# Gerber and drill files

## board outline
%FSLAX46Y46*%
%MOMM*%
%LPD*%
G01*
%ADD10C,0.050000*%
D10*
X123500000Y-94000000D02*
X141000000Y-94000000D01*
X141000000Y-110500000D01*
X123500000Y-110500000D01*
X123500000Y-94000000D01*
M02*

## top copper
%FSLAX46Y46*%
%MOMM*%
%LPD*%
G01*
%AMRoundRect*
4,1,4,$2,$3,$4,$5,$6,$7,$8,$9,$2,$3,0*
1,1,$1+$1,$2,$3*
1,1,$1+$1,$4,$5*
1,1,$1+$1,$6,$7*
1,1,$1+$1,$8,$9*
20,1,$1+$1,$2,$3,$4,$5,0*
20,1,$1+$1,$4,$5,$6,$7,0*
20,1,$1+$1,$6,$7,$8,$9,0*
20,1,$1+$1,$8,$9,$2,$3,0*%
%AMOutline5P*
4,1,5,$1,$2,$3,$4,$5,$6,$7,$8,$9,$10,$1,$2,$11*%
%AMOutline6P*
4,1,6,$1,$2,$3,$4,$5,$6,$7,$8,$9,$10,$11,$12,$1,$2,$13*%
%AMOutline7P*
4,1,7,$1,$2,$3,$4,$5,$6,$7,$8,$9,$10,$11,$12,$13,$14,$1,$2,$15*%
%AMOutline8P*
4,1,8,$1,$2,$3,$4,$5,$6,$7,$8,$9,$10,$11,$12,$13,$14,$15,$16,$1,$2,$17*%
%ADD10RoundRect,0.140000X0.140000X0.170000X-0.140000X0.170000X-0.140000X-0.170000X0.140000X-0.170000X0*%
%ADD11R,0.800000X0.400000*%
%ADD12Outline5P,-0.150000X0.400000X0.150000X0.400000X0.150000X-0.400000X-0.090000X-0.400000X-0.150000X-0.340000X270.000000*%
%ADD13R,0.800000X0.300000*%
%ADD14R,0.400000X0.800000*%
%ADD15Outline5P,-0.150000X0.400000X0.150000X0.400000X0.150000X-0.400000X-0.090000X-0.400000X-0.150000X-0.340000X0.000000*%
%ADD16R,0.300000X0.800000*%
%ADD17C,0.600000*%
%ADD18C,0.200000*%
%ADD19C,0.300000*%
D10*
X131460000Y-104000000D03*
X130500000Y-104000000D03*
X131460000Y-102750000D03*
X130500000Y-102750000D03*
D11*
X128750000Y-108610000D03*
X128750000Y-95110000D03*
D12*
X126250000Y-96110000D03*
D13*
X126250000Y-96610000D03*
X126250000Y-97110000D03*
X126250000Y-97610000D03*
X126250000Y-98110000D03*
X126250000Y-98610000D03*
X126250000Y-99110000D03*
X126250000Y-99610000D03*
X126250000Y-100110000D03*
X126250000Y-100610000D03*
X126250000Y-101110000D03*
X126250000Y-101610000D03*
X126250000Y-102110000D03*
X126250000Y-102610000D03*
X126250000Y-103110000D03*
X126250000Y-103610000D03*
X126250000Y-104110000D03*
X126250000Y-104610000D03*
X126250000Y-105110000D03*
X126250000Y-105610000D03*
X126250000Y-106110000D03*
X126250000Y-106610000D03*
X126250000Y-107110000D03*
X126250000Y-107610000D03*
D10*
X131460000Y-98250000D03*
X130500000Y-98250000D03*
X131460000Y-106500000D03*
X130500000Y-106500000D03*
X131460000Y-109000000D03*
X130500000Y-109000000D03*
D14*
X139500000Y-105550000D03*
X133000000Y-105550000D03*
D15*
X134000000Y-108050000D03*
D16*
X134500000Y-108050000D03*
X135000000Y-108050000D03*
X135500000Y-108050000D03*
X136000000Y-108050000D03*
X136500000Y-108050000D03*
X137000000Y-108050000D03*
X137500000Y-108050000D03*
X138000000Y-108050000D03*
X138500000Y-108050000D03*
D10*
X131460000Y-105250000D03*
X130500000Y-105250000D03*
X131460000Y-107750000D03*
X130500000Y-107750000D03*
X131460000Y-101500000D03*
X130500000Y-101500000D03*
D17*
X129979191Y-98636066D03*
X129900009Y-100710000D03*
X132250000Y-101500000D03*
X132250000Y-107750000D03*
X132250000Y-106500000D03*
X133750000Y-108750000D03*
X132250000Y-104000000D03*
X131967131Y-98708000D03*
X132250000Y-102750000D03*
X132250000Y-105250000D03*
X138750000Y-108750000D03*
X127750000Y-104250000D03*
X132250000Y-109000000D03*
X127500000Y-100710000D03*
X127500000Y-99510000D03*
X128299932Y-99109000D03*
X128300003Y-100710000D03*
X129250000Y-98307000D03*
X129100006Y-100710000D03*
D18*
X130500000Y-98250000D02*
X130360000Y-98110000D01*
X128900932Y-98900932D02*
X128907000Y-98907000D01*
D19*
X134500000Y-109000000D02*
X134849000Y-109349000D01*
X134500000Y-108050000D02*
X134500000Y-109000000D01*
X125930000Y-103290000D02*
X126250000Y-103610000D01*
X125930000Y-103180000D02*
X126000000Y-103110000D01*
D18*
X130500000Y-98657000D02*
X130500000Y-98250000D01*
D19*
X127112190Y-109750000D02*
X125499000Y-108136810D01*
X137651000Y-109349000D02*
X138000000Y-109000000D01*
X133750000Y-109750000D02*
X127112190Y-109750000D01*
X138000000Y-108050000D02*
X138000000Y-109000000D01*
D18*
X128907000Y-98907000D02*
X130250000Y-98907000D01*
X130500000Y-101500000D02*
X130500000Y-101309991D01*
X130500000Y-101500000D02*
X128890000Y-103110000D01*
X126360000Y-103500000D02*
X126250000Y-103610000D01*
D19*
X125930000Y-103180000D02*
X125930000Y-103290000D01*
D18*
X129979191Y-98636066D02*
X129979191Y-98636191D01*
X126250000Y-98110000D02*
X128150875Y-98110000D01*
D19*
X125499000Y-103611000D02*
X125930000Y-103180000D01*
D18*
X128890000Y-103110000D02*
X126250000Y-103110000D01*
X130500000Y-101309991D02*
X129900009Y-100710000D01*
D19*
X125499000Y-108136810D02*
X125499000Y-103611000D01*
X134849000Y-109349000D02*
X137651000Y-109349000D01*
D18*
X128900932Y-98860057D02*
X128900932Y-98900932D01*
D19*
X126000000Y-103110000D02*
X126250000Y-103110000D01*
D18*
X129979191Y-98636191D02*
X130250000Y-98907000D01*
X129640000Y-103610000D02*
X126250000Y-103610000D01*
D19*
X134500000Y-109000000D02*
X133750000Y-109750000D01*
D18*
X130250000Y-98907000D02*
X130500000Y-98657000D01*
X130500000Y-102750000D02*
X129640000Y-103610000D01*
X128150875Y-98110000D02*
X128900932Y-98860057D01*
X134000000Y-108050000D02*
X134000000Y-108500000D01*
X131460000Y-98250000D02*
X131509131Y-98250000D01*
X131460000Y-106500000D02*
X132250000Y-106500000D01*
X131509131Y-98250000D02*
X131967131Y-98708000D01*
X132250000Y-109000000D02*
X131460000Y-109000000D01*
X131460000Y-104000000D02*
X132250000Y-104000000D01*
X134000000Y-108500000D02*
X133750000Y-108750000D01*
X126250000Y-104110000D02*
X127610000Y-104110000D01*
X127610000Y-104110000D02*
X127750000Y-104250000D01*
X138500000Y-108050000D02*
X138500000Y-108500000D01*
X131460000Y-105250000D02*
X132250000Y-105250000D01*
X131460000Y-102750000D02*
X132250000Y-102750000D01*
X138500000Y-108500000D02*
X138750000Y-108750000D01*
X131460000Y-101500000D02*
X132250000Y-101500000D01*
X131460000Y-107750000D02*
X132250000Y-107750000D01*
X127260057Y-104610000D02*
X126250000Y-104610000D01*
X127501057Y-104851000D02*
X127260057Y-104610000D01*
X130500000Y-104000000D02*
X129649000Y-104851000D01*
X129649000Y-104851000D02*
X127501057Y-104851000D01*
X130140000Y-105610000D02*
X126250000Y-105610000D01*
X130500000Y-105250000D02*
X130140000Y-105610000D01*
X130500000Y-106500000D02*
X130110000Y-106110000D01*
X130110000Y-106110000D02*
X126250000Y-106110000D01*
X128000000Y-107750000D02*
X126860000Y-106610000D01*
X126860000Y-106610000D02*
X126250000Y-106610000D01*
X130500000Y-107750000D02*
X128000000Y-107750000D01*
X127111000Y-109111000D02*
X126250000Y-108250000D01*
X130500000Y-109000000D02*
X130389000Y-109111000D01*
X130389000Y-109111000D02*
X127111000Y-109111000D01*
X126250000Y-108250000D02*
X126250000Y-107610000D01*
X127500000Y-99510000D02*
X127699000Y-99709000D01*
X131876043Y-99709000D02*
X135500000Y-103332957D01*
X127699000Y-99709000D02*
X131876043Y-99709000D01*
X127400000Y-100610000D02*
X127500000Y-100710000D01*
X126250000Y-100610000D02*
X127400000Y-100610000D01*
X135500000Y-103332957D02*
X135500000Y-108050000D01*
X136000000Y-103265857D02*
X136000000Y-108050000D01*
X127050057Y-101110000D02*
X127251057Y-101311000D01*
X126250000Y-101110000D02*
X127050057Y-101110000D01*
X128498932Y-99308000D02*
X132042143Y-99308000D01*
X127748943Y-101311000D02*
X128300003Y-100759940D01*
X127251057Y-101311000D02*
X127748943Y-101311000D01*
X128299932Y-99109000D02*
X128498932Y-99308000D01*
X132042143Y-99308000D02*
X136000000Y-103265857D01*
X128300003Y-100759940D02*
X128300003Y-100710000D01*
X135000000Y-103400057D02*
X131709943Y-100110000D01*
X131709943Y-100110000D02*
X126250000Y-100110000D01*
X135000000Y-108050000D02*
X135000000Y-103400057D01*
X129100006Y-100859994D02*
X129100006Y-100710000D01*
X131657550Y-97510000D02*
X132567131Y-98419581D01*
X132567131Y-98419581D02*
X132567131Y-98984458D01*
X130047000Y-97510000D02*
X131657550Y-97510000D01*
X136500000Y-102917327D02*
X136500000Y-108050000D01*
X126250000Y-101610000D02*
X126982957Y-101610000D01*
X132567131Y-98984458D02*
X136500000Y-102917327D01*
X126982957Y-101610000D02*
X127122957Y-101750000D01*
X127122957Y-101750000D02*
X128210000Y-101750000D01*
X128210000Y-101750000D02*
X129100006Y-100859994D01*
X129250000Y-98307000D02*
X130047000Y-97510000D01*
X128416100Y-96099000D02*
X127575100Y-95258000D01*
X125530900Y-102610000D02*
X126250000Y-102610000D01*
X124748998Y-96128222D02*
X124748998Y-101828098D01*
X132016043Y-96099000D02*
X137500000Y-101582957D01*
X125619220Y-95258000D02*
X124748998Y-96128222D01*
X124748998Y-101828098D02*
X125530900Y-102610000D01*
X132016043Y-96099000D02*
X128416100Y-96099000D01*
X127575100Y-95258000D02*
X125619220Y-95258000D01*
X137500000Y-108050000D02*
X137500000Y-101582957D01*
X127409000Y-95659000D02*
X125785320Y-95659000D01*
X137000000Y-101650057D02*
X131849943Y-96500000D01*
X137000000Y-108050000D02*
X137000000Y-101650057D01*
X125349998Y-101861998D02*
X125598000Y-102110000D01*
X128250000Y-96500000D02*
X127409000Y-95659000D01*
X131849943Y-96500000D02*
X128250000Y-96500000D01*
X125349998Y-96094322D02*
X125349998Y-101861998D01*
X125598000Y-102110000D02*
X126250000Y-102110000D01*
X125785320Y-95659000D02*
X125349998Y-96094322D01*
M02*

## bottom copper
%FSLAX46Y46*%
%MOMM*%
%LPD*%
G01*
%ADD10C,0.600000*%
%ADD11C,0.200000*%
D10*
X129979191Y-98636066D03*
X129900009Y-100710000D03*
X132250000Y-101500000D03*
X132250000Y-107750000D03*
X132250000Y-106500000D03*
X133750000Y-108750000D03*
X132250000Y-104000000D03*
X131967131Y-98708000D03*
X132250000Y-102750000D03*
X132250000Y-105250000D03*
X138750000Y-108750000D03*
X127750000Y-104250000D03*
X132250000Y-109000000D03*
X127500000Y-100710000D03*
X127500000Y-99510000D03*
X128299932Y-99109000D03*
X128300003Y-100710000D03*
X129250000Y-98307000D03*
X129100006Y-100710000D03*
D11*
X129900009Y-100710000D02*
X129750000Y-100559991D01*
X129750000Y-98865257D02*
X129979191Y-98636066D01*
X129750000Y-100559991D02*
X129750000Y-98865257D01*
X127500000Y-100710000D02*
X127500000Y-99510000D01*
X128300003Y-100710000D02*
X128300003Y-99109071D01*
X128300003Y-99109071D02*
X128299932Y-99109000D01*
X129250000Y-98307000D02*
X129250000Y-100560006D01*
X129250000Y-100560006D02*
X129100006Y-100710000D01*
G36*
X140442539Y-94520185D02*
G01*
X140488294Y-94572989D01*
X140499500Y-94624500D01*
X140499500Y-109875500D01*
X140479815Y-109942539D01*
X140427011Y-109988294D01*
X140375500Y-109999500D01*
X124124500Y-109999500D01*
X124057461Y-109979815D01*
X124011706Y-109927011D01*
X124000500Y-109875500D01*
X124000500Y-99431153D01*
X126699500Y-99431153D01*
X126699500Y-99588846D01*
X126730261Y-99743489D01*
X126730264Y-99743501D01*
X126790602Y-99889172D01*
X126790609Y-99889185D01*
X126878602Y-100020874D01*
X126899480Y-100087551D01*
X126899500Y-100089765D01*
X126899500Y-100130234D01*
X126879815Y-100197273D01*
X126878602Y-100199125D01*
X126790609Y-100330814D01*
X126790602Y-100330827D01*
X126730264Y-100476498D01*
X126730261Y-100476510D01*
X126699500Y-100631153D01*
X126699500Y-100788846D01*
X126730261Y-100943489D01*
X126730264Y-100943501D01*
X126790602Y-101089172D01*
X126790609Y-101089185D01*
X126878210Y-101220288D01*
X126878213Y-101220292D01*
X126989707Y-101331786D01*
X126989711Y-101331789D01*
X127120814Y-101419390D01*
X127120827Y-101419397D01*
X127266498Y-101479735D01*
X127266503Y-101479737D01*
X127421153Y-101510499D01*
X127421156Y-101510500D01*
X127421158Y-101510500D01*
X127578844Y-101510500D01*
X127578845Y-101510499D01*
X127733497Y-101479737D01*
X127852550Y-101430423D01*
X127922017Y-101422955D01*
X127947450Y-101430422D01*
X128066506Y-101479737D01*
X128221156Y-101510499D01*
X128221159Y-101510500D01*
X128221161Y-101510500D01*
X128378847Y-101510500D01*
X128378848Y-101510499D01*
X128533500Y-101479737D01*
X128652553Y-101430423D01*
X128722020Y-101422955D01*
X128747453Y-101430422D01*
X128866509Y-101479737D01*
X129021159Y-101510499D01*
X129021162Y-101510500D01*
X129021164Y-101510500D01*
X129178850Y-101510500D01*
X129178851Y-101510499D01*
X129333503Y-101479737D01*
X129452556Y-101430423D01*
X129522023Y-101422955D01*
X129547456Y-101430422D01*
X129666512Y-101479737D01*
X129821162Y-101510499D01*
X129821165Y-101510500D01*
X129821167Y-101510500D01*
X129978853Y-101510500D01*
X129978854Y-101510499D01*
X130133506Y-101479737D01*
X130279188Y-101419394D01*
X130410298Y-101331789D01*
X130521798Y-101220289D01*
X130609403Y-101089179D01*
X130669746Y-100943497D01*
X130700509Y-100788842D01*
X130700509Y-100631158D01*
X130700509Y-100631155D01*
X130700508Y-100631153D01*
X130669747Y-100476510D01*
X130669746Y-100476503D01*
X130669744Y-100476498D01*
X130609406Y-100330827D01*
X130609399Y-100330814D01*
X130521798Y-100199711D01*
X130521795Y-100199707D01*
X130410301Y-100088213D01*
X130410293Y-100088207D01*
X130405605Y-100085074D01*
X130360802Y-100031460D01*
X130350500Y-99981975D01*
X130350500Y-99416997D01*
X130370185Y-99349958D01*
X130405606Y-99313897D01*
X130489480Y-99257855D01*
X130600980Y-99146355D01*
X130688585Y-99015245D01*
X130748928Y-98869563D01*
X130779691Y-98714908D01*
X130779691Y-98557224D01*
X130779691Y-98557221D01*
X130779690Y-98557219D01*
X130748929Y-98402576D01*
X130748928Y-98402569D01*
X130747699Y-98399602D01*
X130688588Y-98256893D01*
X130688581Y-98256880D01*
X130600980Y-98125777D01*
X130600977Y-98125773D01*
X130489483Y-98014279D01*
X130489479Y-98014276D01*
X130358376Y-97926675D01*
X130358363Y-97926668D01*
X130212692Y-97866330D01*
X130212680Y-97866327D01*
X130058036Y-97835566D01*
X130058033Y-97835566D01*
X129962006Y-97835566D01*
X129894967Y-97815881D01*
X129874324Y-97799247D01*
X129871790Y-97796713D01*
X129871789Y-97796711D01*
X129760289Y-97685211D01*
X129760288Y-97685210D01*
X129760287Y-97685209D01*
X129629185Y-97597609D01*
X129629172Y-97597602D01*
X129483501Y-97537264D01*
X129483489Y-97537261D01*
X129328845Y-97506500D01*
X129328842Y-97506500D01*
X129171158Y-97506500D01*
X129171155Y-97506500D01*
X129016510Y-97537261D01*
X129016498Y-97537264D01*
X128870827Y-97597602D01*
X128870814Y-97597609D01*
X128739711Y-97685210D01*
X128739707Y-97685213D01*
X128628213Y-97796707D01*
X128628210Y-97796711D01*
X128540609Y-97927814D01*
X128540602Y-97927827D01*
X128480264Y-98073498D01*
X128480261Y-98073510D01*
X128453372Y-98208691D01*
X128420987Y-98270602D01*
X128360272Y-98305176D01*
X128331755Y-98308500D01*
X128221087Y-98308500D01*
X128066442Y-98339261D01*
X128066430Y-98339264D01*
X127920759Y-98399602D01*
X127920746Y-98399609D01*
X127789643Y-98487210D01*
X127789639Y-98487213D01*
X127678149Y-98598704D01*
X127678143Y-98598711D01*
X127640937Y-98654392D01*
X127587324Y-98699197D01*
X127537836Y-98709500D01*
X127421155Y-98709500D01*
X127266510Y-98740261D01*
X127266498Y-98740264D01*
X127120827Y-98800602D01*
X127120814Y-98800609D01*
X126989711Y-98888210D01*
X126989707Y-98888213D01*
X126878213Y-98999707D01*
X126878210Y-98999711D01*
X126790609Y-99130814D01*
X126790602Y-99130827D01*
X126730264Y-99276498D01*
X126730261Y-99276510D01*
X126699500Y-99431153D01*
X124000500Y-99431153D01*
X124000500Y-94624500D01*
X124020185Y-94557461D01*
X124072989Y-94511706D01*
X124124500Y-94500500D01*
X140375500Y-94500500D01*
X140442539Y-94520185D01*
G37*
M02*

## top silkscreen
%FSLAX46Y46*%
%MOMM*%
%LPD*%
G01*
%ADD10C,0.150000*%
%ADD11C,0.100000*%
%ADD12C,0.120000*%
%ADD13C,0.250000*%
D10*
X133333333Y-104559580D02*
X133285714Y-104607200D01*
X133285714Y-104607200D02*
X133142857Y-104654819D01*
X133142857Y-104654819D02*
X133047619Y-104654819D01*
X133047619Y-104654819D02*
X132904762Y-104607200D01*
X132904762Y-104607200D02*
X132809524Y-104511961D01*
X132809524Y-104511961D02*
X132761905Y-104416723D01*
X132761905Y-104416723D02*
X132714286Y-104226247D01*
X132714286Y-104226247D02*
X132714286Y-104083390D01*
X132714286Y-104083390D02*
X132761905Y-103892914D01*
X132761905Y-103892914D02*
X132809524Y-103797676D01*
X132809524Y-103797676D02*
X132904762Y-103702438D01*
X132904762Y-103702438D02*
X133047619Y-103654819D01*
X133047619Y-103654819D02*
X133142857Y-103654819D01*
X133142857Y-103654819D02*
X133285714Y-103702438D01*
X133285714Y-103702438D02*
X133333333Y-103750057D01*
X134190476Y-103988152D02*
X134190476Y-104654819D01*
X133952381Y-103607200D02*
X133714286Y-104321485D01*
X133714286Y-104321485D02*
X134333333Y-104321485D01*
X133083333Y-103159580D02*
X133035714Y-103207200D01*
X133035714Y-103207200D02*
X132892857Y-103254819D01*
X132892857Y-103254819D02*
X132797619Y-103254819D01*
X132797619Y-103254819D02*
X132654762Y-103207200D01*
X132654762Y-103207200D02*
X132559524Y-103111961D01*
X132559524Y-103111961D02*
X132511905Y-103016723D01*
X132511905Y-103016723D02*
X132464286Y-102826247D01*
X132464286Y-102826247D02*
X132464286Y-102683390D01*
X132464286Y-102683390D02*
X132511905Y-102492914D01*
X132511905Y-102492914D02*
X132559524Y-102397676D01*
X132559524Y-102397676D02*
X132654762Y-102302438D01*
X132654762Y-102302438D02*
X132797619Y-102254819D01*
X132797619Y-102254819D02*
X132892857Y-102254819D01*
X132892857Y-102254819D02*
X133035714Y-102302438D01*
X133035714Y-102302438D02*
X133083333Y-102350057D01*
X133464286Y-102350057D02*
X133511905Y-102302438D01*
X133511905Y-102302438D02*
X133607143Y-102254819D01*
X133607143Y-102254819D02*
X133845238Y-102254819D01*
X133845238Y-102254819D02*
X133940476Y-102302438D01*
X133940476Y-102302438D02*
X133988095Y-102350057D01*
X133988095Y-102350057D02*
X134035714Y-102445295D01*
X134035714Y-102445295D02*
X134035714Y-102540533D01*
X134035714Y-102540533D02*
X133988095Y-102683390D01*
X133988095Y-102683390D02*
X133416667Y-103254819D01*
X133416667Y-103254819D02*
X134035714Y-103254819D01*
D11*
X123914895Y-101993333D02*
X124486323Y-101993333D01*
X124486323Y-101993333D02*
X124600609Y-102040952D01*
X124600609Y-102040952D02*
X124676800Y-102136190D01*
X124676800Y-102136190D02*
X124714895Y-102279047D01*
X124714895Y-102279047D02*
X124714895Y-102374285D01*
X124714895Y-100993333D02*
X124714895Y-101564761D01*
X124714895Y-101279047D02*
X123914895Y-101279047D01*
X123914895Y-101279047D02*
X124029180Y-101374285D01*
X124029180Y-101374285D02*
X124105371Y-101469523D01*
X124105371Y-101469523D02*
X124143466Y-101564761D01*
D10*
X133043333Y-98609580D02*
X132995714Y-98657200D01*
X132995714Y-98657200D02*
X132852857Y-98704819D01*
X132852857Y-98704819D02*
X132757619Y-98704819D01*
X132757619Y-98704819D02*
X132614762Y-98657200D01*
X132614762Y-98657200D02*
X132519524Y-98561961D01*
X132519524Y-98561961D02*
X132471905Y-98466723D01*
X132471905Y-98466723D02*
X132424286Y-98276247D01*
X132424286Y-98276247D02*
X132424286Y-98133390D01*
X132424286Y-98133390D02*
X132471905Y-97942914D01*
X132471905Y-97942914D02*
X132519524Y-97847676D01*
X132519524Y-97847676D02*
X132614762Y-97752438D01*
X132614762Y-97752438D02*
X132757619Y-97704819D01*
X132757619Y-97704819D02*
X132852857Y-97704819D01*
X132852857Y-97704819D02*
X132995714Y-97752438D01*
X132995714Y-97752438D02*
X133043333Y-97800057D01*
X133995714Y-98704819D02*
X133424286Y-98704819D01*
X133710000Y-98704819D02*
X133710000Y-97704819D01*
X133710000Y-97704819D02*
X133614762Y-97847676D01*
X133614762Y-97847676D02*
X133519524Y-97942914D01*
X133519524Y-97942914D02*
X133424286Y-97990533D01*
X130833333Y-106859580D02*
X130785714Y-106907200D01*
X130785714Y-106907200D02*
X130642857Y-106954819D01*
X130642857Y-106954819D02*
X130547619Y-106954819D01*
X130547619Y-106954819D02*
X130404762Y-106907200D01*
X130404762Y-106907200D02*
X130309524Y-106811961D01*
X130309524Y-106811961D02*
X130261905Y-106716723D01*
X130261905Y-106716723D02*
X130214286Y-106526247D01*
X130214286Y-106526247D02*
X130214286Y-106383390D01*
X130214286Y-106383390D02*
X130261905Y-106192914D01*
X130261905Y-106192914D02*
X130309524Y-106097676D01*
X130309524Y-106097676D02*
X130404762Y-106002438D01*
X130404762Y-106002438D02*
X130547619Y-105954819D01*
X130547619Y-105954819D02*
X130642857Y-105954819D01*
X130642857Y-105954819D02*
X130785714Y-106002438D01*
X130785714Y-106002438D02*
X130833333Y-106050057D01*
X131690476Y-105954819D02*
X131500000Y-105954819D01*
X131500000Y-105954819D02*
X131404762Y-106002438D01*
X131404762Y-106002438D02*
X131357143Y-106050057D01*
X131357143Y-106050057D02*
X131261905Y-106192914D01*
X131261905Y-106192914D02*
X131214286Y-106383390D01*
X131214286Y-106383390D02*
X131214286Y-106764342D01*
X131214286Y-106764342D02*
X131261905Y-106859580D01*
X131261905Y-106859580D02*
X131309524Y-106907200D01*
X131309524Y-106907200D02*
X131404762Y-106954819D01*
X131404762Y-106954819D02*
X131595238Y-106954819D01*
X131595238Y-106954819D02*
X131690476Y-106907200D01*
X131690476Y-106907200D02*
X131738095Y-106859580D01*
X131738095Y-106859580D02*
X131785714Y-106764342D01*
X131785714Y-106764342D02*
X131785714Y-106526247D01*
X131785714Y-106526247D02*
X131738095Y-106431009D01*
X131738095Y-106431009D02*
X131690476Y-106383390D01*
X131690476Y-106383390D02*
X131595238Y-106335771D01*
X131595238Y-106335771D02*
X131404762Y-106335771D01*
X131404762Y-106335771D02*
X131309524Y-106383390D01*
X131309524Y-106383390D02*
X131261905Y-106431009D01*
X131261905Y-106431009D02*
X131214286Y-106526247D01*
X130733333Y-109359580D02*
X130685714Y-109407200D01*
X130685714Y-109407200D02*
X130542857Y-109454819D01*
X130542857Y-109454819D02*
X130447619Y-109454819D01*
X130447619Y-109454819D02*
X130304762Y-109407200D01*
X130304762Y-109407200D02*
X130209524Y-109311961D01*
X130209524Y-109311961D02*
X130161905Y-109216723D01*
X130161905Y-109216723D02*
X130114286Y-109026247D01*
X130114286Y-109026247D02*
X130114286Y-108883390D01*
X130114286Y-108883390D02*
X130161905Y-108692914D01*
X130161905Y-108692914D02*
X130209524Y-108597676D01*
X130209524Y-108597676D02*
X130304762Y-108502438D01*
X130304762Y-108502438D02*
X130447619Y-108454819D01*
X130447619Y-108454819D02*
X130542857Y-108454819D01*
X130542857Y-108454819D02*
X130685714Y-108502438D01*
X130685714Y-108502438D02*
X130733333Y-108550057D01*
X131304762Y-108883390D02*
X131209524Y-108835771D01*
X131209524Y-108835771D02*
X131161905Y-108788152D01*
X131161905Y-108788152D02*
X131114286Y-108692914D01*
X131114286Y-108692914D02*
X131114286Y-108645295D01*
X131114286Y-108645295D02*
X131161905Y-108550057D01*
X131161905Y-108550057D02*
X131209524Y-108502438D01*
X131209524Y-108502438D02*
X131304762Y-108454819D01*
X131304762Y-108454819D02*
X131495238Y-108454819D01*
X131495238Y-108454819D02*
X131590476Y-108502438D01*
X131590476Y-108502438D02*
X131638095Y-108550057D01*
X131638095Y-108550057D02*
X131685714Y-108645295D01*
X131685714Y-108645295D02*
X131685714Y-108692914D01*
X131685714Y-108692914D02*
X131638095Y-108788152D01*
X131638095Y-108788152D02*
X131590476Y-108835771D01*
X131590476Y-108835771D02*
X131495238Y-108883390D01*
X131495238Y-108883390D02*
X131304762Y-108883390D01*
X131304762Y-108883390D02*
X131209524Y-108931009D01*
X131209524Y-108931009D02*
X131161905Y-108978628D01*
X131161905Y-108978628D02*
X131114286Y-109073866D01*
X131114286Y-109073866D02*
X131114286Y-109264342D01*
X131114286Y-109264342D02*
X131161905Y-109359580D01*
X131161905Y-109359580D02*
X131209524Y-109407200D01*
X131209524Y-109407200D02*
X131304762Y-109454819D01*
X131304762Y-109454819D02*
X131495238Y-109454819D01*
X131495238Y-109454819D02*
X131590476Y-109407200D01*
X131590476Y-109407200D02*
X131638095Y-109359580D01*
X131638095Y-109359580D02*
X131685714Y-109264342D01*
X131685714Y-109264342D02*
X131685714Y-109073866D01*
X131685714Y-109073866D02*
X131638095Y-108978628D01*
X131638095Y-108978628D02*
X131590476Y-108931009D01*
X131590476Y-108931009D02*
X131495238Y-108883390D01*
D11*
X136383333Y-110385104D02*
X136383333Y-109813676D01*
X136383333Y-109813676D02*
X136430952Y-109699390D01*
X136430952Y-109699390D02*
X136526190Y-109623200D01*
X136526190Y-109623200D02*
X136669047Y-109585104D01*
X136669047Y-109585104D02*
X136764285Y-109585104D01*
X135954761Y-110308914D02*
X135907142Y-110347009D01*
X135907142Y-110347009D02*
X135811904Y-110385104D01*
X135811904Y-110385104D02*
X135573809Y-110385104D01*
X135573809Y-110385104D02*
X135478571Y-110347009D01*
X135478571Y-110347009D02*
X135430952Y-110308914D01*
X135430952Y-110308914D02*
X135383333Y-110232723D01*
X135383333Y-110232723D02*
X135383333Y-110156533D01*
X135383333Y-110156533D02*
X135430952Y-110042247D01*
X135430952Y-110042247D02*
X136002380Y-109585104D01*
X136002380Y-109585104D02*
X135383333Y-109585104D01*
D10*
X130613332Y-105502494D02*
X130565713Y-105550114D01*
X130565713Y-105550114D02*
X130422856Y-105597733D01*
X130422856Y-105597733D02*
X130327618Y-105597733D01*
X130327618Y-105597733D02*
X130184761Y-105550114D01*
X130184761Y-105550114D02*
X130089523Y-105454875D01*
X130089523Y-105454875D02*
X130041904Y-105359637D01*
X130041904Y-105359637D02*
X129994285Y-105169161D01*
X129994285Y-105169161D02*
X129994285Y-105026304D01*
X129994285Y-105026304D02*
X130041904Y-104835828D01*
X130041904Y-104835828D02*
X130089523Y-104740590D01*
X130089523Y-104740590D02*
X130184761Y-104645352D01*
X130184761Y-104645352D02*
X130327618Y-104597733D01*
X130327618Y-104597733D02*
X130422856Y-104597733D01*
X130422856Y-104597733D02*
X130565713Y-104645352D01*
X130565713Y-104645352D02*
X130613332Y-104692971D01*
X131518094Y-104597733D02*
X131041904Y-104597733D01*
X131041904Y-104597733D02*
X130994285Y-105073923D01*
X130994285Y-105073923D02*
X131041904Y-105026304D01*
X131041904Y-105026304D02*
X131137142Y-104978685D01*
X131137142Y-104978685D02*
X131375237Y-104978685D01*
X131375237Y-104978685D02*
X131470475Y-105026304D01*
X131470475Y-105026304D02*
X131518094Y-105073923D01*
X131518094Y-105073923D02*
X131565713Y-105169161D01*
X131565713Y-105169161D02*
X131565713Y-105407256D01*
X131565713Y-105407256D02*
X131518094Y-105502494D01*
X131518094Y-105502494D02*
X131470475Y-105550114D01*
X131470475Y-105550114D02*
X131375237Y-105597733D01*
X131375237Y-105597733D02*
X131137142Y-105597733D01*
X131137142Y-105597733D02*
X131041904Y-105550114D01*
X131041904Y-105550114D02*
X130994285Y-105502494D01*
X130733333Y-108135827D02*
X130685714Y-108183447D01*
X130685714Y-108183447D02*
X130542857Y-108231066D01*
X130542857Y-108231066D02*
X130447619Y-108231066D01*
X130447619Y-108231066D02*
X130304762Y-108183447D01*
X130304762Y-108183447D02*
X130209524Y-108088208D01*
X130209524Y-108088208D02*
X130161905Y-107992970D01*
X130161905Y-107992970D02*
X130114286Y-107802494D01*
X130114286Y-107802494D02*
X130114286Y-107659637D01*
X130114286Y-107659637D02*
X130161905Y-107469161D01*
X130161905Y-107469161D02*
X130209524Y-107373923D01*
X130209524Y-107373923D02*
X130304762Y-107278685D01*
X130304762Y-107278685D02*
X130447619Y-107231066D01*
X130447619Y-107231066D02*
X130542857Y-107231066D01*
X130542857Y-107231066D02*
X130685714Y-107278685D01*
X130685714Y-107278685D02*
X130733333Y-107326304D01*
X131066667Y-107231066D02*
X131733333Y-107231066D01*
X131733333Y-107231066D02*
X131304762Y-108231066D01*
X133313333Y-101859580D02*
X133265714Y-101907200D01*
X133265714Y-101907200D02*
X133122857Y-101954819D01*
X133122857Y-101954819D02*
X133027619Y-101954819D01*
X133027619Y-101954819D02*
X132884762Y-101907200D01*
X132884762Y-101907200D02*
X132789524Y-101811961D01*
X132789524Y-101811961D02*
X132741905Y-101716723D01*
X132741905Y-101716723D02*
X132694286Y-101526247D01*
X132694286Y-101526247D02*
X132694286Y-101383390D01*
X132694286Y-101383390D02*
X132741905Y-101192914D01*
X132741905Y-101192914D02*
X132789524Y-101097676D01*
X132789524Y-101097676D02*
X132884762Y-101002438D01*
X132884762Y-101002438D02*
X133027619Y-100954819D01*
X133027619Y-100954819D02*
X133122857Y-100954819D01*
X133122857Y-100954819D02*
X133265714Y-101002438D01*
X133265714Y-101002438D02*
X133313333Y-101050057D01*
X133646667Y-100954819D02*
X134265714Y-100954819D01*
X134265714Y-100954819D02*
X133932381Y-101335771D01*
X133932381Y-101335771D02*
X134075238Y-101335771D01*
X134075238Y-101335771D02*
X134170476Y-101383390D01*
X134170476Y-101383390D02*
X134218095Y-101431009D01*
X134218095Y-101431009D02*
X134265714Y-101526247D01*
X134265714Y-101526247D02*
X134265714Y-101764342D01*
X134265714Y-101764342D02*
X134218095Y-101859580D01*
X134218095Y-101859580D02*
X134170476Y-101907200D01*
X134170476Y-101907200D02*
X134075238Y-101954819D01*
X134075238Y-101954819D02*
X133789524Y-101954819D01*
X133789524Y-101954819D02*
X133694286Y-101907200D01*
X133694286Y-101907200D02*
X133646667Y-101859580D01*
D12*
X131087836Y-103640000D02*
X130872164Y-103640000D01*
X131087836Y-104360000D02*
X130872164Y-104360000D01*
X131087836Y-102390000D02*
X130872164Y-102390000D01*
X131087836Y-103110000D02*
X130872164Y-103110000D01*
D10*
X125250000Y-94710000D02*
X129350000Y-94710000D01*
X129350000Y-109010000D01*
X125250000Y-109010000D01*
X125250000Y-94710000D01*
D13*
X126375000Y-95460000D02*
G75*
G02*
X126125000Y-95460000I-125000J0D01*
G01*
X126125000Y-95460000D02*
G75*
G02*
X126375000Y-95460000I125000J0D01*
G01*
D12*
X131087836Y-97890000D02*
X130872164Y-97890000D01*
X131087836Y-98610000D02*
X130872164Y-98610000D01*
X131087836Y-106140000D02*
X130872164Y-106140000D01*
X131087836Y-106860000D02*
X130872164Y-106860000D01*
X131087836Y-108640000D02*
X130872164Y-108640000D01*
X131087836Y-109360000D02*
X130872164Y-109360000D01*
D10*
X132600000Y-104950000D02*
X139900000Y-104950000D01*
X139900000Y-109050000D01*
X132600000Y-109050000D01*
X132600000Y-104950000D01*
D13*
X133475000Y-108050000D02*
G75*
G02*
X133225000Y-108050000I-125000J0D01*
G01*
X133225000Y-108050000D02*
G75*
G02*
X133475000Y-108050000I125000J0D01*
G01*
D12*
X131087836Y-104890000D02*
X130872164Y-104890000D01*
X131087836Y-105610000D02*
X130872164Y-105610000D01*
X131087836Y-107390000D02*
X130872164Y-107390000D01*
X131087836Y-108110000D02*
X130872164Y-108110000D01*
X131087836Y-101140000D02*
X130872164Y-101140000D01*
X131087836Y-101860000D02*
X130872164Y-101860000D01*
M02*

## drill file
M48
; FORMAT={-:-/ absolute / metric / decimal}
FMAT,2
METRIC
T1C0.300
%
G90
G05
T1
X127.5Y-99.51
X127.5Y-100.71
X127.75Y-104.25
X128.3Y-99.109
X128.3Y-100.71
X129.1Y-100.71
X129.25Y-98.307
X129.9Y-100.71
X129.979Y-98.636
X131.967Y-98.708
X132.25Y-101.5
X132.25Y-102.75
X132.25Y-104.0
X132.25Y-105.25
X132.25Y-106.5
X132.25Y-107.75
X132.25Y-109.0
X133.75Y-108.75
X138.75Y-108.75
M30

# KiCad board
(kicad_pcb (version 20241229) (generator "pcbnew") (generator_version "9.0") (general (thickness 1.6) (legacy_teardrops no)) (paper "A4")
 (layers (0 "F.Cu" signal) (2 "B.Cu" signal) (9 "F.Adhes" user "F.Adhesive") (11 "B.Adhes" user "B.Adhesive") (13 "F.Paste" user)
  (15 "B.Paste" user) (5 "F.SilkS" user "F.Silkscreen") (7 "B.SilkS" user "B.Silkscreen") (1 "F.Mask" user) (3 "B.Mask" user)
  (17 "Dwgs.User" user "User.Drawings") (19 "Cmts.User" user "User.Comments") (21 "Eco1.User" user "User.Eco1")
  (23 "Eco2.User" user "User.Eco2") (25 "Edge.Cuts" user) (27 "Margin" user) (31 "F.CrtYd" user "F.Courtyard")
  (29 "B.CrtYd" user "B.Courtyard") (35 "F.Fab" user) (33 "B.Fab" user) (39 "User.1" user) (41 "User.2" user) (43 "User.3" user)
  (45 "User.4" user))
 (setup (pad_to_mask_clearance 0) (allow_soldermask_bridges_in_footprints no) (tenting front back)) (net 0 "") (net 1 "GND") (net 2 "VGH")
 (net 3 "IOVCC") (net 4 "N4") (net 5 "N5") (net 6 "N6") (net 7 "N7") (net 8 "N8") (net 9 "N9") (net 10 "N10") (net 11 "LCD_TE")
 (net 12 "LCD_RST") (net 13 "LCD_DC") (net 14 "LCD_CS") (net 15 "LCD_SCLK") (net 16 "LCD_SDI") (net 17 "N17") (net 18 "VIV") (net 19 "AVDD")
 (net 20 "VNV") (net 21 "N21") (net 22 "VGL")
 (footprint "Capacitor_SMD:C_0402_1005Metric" (layer "F.Cu") (at 130.98 104 180)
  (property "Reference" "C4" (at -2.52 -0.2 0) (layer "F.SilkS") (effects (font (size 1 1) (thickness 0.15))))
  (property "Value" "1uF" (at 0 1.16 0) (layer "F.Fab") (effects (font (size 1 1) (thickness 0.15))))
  (fp_line (start -0.107836 0.36) (end 0.107836 0.36) (stroke (width 0.12) (type solid)) (layer "F.SilkS"))
  (fp_line (start -0.107836 -0.36) (end 0.107836 -0.36) (stroke (width 0.12) (type solid)) (layer "F.SilkS"))
  (pad "1" smd roundrect (at -0.48 0 180) (size 0.56 0.62) (layers "F.Cu" "F.Mask" "F.Paste") (roundrect_rratio 0.25) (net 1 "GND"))
  (pad "2" smd roundrect (at 0.48 0 180) (size 0.56 0.62) (layers "F.Cu" "F.Mask" "F.Paste") (roundrect_rratio 0.25) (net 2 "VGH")))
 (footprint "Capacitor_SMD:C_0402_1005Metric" (layer "F.Cu") (at 130.98 102.75 180)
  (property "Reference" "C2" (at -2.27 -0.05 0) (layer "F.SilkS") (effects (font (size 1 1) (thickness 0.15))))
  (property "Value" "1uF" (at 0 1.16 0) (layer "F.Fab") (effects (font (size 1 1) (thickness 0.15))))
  (fp_line (start -0.107836 0.36) (end 0.107836 0.36) (stroke (width 0.12) (type solid)) (layer "F.SilkS"))
  (fp_line (start -0.107836 -0.36) (end 0.107836 -0.36) (stroke (width 0.12) (type solid)) (layer "F.SilkS"))
  (pad "1" smd roundrect (at -0.48 0 180) (size 0.56 0.62) (layers "F.Cu" "F.Mask" "F.Paste") (roundrect_rratio 0.25) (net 1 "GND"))
  (pad "2" smd roundrect (at 0.48 0 180) (size 0.56 0.62) (layers "F.Cu" "F.Mask" "F.Paste") (roundrect_rratio 0.25) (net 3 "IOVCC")))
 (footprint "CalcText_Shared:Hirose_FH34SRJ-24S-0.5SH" (layer "F.Cu") (at 126.25 101.86 90)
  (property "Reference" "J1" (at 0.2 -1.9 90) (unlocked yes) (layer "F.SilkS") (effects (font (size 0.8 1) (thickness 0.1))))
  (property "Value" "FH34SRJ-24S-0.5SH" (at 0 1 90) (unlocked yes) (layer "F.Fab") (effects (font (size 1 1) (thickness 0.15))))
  (fp_rect (start -7.15 -1) (end 7.15 3.1) (stroke (width 0.15) (type solid)) (fill no) (layer "F.SilkS"))
  (fp_circle (center 6.4 0) (end 6.6 0) (stroke (width 0.1) (type default)) (fill yes) (layer "F.SilkS"))
  (pad "" smd rect (at -6.75 2.5 90) (size 0.4 0.8) (layers "F.Cu" "F.Mask" "F.Paste") (thermal_bridge_angle 45))
  (pad "" smd rect (at 6.75 2.5 90) (size 0.4 0.8) (layers "F.Cu" "F.Mask" "F.Paste") (thermal_bridge_angle 45))
  (pad "1" smd roundrect (at 5.75 0 270) (size 0.3 0.8) (layers "F.Cu" "F.Mask" "F.Paste") (roundrect_rratio 0) (chamfer_ratio 0.2)
   (chamfer bottom_left) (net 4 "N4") (thermal_bridge_angle 45))
  (pad "2" smd rect (at 5.25 0 270) (size 0.3 0.8) (layers "F.Cu" "F.Mask" "F.Paste") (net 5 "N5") (thermal_bridge_angle 45))
  (pad "3" smd rect (at 4.75 0 270) (size 0.3 0.8) (layers "F.Cu" "F.Mask" "F.Paste") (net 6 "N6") (thermal_bridge_angle 45))
  (pad "4" smd rect (at 4.25 0 270) (size 0.3 0.8) (layers "F.Cu" "F.Mask" "F.Paste") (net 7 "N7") (thermal_bridge_angle 45))
  (pad "5" smd rect (at 3.75 0 270) (size 0.3 0.8) (layers "F.Cu" "F.Mask" "F.Paste") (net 3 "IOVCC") (thermal_bridge_angle 45))
  (pad "6" smd rect (at 3.25 0 270) (size 0.3 0.8) (layers "F.Cu" "F.Mask" "F.Paste") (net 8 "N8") (thermal_bridge_angle 45))
  (pad "7" smd rect (at 2.75 0 270) (size 0.3 0.8) (layers "F.Cu" "F.Mask" "F.Paste") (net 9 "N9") (thermal_bridge_angle 45))
  (pad "8" smd rect (at 2.25 0 270) (size 0.3 0.8) (layers "F.Cu" "F.Mask" "F.Paste") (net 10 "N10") (thermal_bridge_angle 45))
  (pad "9" smd rect (at 1.75 0 270) (size 0.3 0.8) (layers "F.Cu" "F.Mask" "F.Paste") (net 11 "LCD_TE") (thermal_bridge_angle 45))
  (pad "10" smd rect (at 1.25 0 270) (size 0.3 0.8) (layers "F.Cu" "F.Mask" "F.Paste") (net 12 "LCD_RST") (thermal_bridge_angle 45))
  (pad "11" smd rect (at 0.75 0 270) (size 0.3 0.8) (layers "F.Cu" "F.Mask" "F.Paste") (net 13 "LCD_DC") (thermal_bridge_angle 45))
  (pad "12" smd rect (at 0.25 0 270) (size 0.3 0.8) (layers "F.Cu" "F.Mask" "F.Paste") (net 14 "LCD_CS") (thermal_bridge_angle 45))
  (pad "13" smd rect (at -0.25 0 270) (size 0.3 0.8) (layers "F.Cu" "F.Mask" "F.Paste") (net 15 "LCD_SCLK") (thermal_bridge_angle 45))
  (pad "14" smd rect (at -0.75 0 270) (size 0.3 0.8) (layers "F.Cu" "F.Mask" "F.Paste") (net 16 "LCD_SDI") (thermal_bridge_angle 45))
  (pad "15" smd rect (at -1.25 0 270) (size 0.3 0.8) (layers "F.Cu" "F.Mask" "F.Paste") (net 3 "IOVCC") (thermal_bridge_angle 45))
  (pad "16" smd rect (at -1.75 0 270) (size 0.3 0.8) (layers "F.Cu" "F.Mask" "F.Paste") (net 3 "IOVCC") (thermal_bridge_angle 45))
  (pad "17" smd rect (at -2.25 0 270) (size 0.3 0.8) (layers "F.Cu" "F.Mask" "F.Paste") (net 1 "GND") (thermal_bridge_angle 45))
  (pad "18" smd rect (at -2.75 0 270) (size 0.3 0.8) (layers "F.Cu" "F.Mask" "F.Paste") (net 2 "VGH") (thermal_bridge_angle 45))
  (pad "19" smd rect (at -3.25 0 270) (size 0.3 0.8) (layers "F.Cu" "F.Mask" "F.Paste") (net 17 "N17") (thermal_bridge_angle 45))
  (pad "20" smd rect (at -3.75 0 270) (size 0.3 0.8) (layers "F.Cu" "F.Mask" "F.Paste") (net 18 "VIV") (thermal_bridge_angle 45))
  (pad "21" smd rect (at -4.25 0 270) (size 0.3 0.8) (layers "F.Cu" "F.Mask" "F.Paste") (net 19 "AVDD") (thermal_bridge_angle 45))
  (pad "22" smd rect (at -4.75 0 270) (size 0.3 0.8) (layers "F.Cu" "F.Mask" "F.Paste") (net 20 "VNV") (thermal_bridge_angle 45))
  (pad "23" smd rect (at -5.25 0 270) (size 0.3 0.8) (layers "F.Cu" "F.Mask" "F.Paste") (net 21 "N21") (thermal_bridge_angle 45))
  (pad "24" smd rect (at -5.75 0 270) (size 0.3 0.8) (layers "F.Cu" "F.Mask" "F.Paste") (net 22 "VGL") (thermal_bridge_angle 45)))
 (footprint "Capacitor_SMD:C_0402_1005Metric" (layer "F.Cu") (at 130.98 98.25 180)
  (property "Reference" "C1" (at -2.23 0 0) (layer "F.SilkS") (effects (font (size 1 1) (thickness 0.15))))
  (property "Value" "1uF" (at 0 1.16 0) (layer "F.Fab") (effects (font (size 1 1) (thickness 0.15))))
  (fp_line (start -0.107836 0.36) (end 0.107836 0.36) (stroke (width 0.12) (type solid)) (layer "F.SilkS"))
  (fp_line (start -0.107836 -0.36) (end 0.107836 -0.36) (stroke (width 0.12) (type solid)) (layer "F.SilkS"))
  (pad "1" smd roundrect (at -0.48 0 180) (size 0.56 0.62) (layers "F.Cu" "F.Mask" "F.Paste") (roundrect_rratio 0.25) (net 1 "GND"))
  (pad "2" smd roundrect (at 0.48 0 180) (size 0.56 0.62) (layers "F.Cu" "F.Mask" "F.Paste") (roundrect_rratio 0.25) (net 3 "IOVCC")))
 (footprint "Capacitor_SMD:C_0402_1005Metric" (layer "F.Cu") (at 130.98 106.5 180)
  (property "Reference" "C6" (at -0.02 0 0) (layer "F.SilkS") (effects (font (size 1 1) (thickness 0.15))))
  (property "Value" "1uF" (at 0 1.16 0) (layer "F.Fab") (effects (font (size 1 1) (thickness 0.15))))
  (fp_line (start -0.107836 0.36) (end 0.107836 0.36) (stroke (width 0.12) (type solid)) (layer "F.SilkS"))
  (fp_line (start -0.107836 -0.36) (end 0.107836 -0.36) (stroke (width 0.12) (type solid)) (layer "F.SilkS"))
  (pad "1" smd roundrect (at -0.48 0 180) (size 0.56 0.62) (layers "F.Cu" "F.Mask" "F.Paste") (roundrect_rratio 0.25) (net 1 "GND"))
  (pad "2" smd roundrect (at 0.48 0 180) (size 0.56 0.62) (layers "F.Cu" "F.Mask" "F.Paste") (roundrect_rratio 0.25) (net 19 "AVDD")))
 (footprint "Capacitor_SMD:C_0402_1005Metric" (layer "F.Cu") (at 130.98 109 180)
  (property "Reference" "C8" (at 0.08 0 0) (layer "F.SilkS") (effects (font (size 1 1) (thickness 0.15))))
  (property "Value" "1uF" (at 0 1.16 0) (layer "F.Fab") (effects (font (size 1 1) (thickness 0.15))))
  (fp_line (start -0.107836 0.36) (end 0.107836 0.36) (stroke (width 0.12) (type solid)) (layer "F.SilkS"))
  (fp_line (start -0.107836 -0.36) (end 0.107836 -0.36) (stroke (width 0.12) (type solid)) (layer "F.SilkS"))
  (pad "1" smd roundrect (at -0.48 0 180) (size 0.56 0.62) (layers "F.Cu" "F.Mask" "F.Paste") (roundrect_rratio 0.25) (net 1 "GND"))
  (pad "2" smd roundrect (at 0.48 0 180) (size 0.56 0.62) (layers "F.Cu" "F.Mask" "F.Paste") (roundrect_rratio 0.25) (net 22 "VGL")))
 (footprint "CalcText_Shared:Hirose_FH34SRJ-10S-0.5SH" (layer "F.Cu") (at 136.25 108.05 180)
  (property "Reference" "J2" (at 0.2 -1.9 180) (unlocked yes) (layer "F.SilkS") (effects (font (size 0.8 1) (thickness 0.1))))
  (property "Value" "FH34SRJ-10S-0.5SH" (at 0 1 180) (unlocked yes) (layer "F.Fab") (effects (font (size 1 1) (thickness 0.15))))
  (fp_rect (start -3.65 -1) (end 3.65 3.1) (stroke (width 0.15) (type solid)) (fill no) (layer "F.SilkS"))
  (fp_circle (center 2.9 0) (end 3.1 0) (stroke (width 0.1) (type default)) (fill yes) (layer "F.SilkS"))
  (pad "" smd rect (at -3.25 2.5 180) (size 0.4 0.8) (layers "F.Cu" "F.Mask" "F.Paste") (thermal_bridge_angle 45))
  (pad "" smd rect (at 3.25 2.5 180) (size 0.4 0.8) (layers "F.Cu" "F.Mask" "F.Paste") (thermal_bridge_angle 45))
  (pad "1" smd roundrect (at 2.25 0) (size 0.3 0.8) (layers "F.Cu" "F.Mask" "F.Paste") (roundrect_rratio 0) (chamfer_ratio 0.2)
   (chamfer bottom_left) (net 1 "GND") (thermal_bridge_angle 45))
  (pad "2" smd rect (at 1.75 0) (size 0.3 0.8) (layers "F.Cu" "F.Mask" "F.Paste") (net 3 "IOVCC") (thermal_bridge_angle 45))
  (pad "3" smd rect (at 1.25 0) (size 0.3 0.8) (layers "F.Cu" "F.Mask" "F.Paste") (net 11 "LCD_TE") (thermal_bridge_angle 45))
  (pad "4" smd rect (at 0.75 0) (size 0.3 0.8) (layers "F.Cu" "F.Mask" "F.Paste") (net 12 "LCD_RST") (thermal_bridge_angle 45))
  (pad "5" smd rect (at 0.25 0) (size 0.3 0.8) (layers "F.Cu" "F.Mask" "F.Paste") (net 13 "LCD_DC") (thermal_bridge_angle 45))
  (pad "6" smd rect (at -0.25 0) (size 0.3 0.8) (layers "F.Cu" "F.Mask" "F.Paste") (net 14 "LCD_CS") (thermal_bridge_angle 45))
  (pad "7" smd rect (at -0.75 0) (size 0.3 0.8) (layers "F.Cu" "F.Mask" "F.Paste") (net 15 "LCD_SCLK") (thermal_bridge_angle 45))
  (pad "8" smd rect (at -1.25 0) (size 0.3 0.8) (layers "F.Cu" "F.Mask" "F.Paste") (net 16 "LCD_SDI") (thermal_bridge_angle 45))
  (pad "9" smd rect (at -1.75 0) (size 0.3 0.8) (layers "F.Cu" "F.Mask" "F.Paste") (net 3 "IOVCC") (thermal_bridge_angle 45))
  (pad "10" smd rect (at -2.25 0) (size 0.3 0.8) (layers "F.Cu" "F.Mask" "F.Paste") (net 1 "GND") (thermal_bridge_angle 45)))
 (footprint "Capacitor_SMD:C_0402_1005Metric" (layer "F.Cu") (at 130.98 105.25 180)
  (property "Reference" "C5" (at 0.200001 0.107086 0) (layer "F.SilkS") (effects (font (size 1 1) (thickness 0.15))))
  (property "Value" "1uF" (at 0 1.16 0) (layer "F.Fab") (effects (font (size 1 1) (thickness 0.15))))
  (fp_line (start -0.107836 0.36) (end 0.107836 0.36) (stroke (width 0.12) (type solid)) (layer "F.SilkS"))
  (fp_line (start -0.107836 -0.36) (end 0.107836 -0.36) (stroke (width 0.12) (type solid)) (layer "F.SilkS"))
  (pad "1" smd roundrect (at -0.48 0 180) (size 0.56 0.62) (layers "F.Cu" "F.Mask" "F.Paste") (roundrect_rratio 0.25) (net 1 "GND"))
  (pad "2" smd roundrect (at 0.48 0 180) (size 0.56 0.62) (layers "F.Cu" "F.Mask" "F.Paste") (roundrect_rratio 0.25) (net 18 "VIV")))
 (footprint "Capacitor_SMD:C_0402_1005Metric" (layer "F.Cu") (at 130.98 107.75 180)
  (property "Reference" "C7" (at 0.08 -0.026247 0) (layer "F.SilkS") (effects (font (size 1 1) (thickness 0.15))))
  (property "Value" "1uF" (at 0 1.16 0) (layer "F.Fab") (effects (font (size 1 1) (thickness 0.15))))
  (fp_line (start -0.107836 0.36) (end 0.107836 0.36) (stroke (width 0.12) (type solid)) (layer "F.SilkS"))
  (fp_line (start -0.107836 -0.36) (end 0.107836 -0.36) (stroke (width 0.12) (type solid)) (layer "F.SilkS"))
  (pad "1" smd roundrect (at -0.48 0 180) (size 0.56 0.62) (layers "F.Cu" "F.Mask" "F.Paste") (roundrect_rratio 0.25) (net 1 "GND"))
  (pad "2" smd roundrect (at 0.48 0 180) (size 0.56 0.62) (layers "F.Cu" "F.Mask" "F.Paste") (roundrect_rratio 0.25) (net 20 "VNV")))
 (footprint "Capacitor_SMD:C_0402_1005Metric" (layer "F.Cu") (at 130.98 101.5 180)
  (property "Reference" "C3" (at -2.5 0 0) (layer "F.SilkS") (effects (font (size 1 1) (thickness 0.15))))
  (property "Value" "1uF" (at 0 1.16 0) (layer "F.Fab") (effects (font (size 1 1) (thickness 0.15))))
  (fp_line (start -0.107836 0.36) (end 0.107836 0.36) (stroke (width 0.12) (type solid)) (layer "F.SilkS"))
  (fp_line (start -0.107836 -0.36) (end 0.107836 -0.36) (stroke (width 0.12) (type solid)) (layer "F.SilkS"))
  (pad "1" smd roundrect (at -0.48 0 180) (size 0.56 0.62) (layers "F.Cu" "F.Mask" "F.Paste") (roundrect_rratio 0.25) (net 1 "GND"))
  (pad "2" smd roundrect (at 0.48 0 180) (size 0.56 0.62) (layers "F.Cu" "F.Mask" "F.Paste") (roundrect_rratio 0.25) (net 3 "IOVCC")))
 (gr_rect (start 123.5 94) (end 141 110.5) (stroke (width 0.05) (type default)) (fill no) (layer "Edge.Cuts"))
 (segment (start 130.5 98.25) (end 130.36 98.11) (width 0.2) (layer "F.Cu") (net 3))
 (segment (start 128.900932 98.900932) (end 128.907 98.907) (width 0.2) (layer "F.Cu") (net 3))
 (segment (start 134.5 109) (end 134.849 109.349) (width 0.3) (layer "F.Cu") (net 3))
 (segment (start 134.5 108.05) (end 134.5 109) (width 0.3) (layer "F.Cu") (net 3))
 (segment (start 125.93 103.29) (end 126.25 103.61) (width 0.3) (layer "F.Cu") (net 3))
 (segment (start 125.93 103.18) (end 126 103.11) (width 0.3) (layer "F.Cu") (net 3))
 (segment (start 130.5 98.657) (end 130.5 98.25) (width 0.2) (layer "F.Cu") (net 3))
 (segment (start 127.11219 109.75) (end 125.499 108.13681) (width 0.3) (layer "F.Cu") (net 3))
 (segment (start 137.651 109.349) (end 138 109) (width 0.3) (layer "F.Cu") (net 3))
 (segment (start 133.75 109.75) (end 127.11219 109.75) (width 0.3) (layer "F.Cu") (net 3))
 (segment (start 138 108.05) (end 138 109) (width 0.3) (layer "F.Cu") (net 3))
 (segment (start 128.907 98.907) (end 130.25 98.907) (width 0.2) (layer "F.Cu") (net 3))
 (segment (start 130.5 101.5) (end 130.5 101.309991) (width 0.2) (layer "F.Cu") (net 3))
 (segment (start 130.5 101.5) (end 128.89 103.11) (width 0.2) (layer "F.Cu") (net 3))
 (segment (start 126.36 103.5) (end 126.25 103.61) (width 0.2) (layer "F.Cu") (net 3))
 (segment (start 125.93 103.18) (end 125.93 103.29) (width 0.3) (layer "F.Cu") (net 3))
 (segment (start 129.979191 98.636066) (end 129.979191 98.636191) (width 0.2) (layer "F.Cu") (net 3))
 (segment (start 126.25 98.11) (end 128.150875 98.11) (width 0.2) (layer "F.Cu") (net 3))
 (segment (start 125.499 103.611) (end 125.93 103.18) (width 0.3) (layer "F.Cu") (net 3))
 (segment (start 128.89 103.11) (end 126.25 103.11) (width 0.2) (layer "F.Cu") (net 3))
 (segment (start 130.5 101.309991) (end 129.900009 100.71) (width 0.2) (layer "F.Cu") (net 3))
 (segment (start 125.499 108.13681) (end 125.499 103.611) (width 0.3) (layer "F.Cu") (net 3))
 (segment (start 134.849 109.349) (end 137.651 109.349) (width 0.3) (layer "F.Cu") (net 3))
 (segment (start 128.900932 98.860057) (end 128.900932 98.900932) (width 0.2) (layer "F.Cu") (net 3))
 (segment (start 126 103.11) (end 126.25 103.11) (width 0.3) (layer "F.Cu") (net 3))
 (segment (start 129.979191 98.636191) (end 130.25 98.907) (width 0.2) (layer "F.Cu") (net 3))
 (segment (start 129.64 103.61) (end 126.25 103.61) (width 0.2) (layer "F.Cu") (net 3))
 (segment (start 134.5 109) (end 133.75 109.75) (width 0.3) (layer "F.Cu") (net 3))
 (segment (start 130.25 98.907) (end 130.5 98.657) (width 0.2) (layer "F.Cu") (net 3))
 (segment (start 130.5 102.75) (end 129.64 103.61) (width 0.2) (layer "F.Cu") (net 3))
 (segment (start 128.150875 98.11) (end 128.900932 98.860057) (width 0.2) (layer "F.Cu") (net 3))
 (via (at 129.979191 98.636066) (size 0.6) (drill 0.3) (layers "F.Cu" "B.Cu") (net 3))
 (via (at 129.900009 100.71) (size 0.6) (drill 0.3) (layers "F.Cu" "B.Cu") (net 3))
 (segment (start 129.900009 100.71) (end 129.75 100.559991) (width 0.2) (layer "B.Cu") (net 3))
 (segment (start 129.75 98.865257) (end 129.979191 98.636066) (width 0.2) (layer "B.Cu") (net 3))
 (segment (start 129.75 100.559991) (end 129.75 98.865257) (width 0.2) (layer "B.Cu") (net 3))
 (segment (start 134 108.05) (end 134 108.5) (width 0.2) (layer "F.Cu") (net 1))
 (segment (start 131.46 98.25) (end 131.509131 98.25) (width 0.2) (layer "F.Cu") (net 1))
 (segment (start 131.46 106.5) (end 132.25 106.5) (width 0.2) (layer "F.Cu") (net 1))
 (segment (start 131.509131 98.25) (end 131.967131 98.708) (width 0.2) (layer "F.Cu") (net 1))
 (segment (start 132.25 109) (end 131.46 109) (width 0.2) (layer "F.Cu") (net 1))
 (segment (start 131.46 104) (end 132.25 104) (width 0.2) (layer "F.Cu") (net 1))
 (segment (start 134 108.5) (end 133.75 108.75) (width 0.2) (layer "F.Cu") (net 1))
 (segment (start 126.25 104.11) (end 127.61 104.11) (width 0.2) (layer "F.Cu") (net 1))
 (segment (start 127.61 104.11) (end 127.75 104.25) (width 0.2) (layer "F.Cu") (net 1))
 (segment (start 138.5 108.05) (end 138.5 108.5) (width 0.2) (layer "F.Cu") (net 1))
 (segment (start 131.46 105.25) (end 132.25 105.25) (width 0.2) (layer "F.Cu") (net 1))
 (segment (start 131.46 102.75) (end 132.25 102.75) (width 0.2) (layer "F.Cu") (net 1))
 (segment (start 138.5 108.5) (end 138.75 108.75) (width 0.2) (layer "F.Cu") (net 1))
 (segment (start 131.46 101.5) (end 132.25 101.5) (width 0.2) (layer "F.Cu") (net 1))
 (segment (start 131.46 107.75) (end 132.25 107.75) (width 0.2) (layer "F.Cu") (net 1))
 (via (at 132.25 101.5) (size 0.6) (drill 0.3) (layers "F.Cu" "B.Cu") (free yes) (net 1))
 (via (at 132.25 107.75) (size 0.6) (drill 0.3) (layers "F.Cu" "B.Cu") (free yes) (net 1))
 (via (at 132.25 106.5) (size 0.6) (drill 0.3) (layers "F.Cu" "B.Cu") (free yes) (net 1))
 (via (at 133.75 108.75) (size 0.6) (drill 0.3) (layers "F.Cu" "B.Cu") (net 1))
 (via (at 132.25 104) (size 0.6) (drill 0.3) (layers "F.Cu" "B.Cu") (free yes) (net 1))
 (via (at 131.967131 98.708) (size 0.6) (drill 0.3) (layers "F.Cu" "B.Cu") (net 1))
 (via (at 132.25 102.75) (size 0.6) (drill 0.3) (layers "F.Cu" "B.Cu") (free yes) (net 1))
 (via (at 132.25 105.25) (size 0.6) (drill 0.3) (layers "F.Cu" "B.Cu") (free yes) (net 1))
 (via (at 138.75 108.75) (size 0.6) (drill 0.3) (layers "F.Cu" "B.Cu") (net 1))
 (via (at 127.75 104.25) (size 0.6) (drill 0.3) (layers "F.Cu" "B.Cu") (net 1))
 (via (at 132.25 109) (size 0.6) (drill 0.3) (layers "F.Cu" "B.Cu") (free yes) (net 1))
 (segment (start 127.260057 104.61) (end 126.25 104.61) (width 0.2) (layer "F.Cu") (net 2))
 (segment (start 127.501057 104.851) (end 127.260057 104.61) (width 0.2) (layer "F.Cu") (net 2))
 (segment (start 130.5 104) (end 129.649 104.851) (width 0.2) (layer "F.Cu") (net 2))
 (segment (start 129.649 104.851) (end 127.501057 104.851) (width 0.2) (layer "F.Cu") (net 2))
 (segment (start 130.14 105.61) (end 126.25 105.61) (width 0.2) (layer "F.Cu") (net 18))
 (segment (start 130.5 105.25) (end 130.14 105.61) (width 0.2) (layer "F.Cu") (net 18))
 (segment (start 130.5 106.5) (end 130.11 106.11) (width 0.2) (layer "F.Cu") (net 19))
 (segment (start 130.11 106.11) (end 126.25 106.11) (width 0.2) (layer "F.Cu") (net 19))
 (segment (start 128 107.75) (end 126.86 106.61) (width 0.2) (layer "F.Cu") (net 20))
 (segment (start 126.86 106.61) (end 126.25 106.61) (width 0.2) (layer "F.Cu") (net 20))
 (segment (start 130.5 107.75) (end 128 107.75) (width 0.2) (layer "F.Cu") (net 20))
 (segment (start 127.111 109.111) (end 126.25 108.25) (width 0.2) (layer "F.Cu") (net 22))
 (segment (start 130.5 109) (end 130.389 109.111) (width 0.2) (layer "F.Cu") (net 22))
 (segment (start 130.389 109.111) (end 127.111 109.111) (width 0.2) (layer "F.Cu") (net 22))
 (segment (start 126.25 108.25) (end 126.25 107.61) (width 0.2) (layer "F.Cu") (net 22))
 (segment (start 127.5 99.51) (end 127.699 99.709) (width 0.2) (layer "F.Cu") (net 12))
 (segment (start 131.876043 99.709) (end 135.5 103.332957) (width 0.2) (layer "F.Cu") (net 12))
 (segment (start 127.699 99.709) (end 131.876043 99.709) (width 0.2) (layer "F.Cu") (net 12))
 (segment (start 127.4 100.61) (end 127.5 100.71) (width 0.2) (layer "F.Cu") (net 12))
 (segment (start 126.25 100.61) (end 127.4 100.61) (width 0.2) (layer "F.Cu") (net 12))
 (segment (start 135.5 103.332957) (end 135.5 108.05) (width 0.2) (layer "F.Cu") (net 12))
 (via (at 127.5 100.71) (size 0.6) (drill 0.3) (layers "F.Cu" "B.Cu") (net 12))
 (via (at 127.5 99.51) (size 0.6) (drill 0.3) (layers "F.Cu" "B.Cu") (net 12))
 (segment (start 127.5 100.71) (end 127.5 99.51) (width 0.2) (layer "B.Cu") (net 12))
 (segment (start 136 103.265857) (end 136 108.05) (width 0.2) (layer "F.Cu") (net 13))
 (segment (start 127.050057 101.11) (end 127.251057 101.311) (width 0.2) (layer "F.Cu") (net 13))
 (segment (start 126.25 101.11) (end 127.050057 101.11) (width 0.2) (layer "F.Cu") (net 13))
 (segment (start 128.498932 99.308) (end 132.042143 99.308) (width 0.2) (layer "F.Cu") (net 13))
 (segment (start 127.748943 101.311) (end 128.300003 100.75994) (width 0.2) (layer "F.Cu") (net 13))
 (segment (start 127.251057 101.311) (end 127.748943 101.311) (width 0.2) (layer "F.Cu") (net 13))
 (segment (start 128.299932 99.109) (end 128.498932 99.308) (width 0.2) (layer "F.Cu") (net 13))
 (segment (start 132.042143 99.308) (end 136 103.265857) (width 0.2) (layer "F.Cu") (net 13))
 (segment (start 128.300003 100.75994) (end 128.300003 100.71) (width 0.2) (layer "F.Cu") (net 13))
 (via (at 128.299932 99.109) (size 0.6) (drill 0.3) (layers "F.Cu" "B.Cu") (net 13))
 (via (at 128.300003 100.71) (size 0.6) (drill 0.3) (layers "F.Cu" "B.Cu") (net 13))
 (segment (start 128.300003 100.71) (end 128.300003 99.109071) (width 0.2) (layer "B.Cu") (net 13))
 (segment (start 128.300003 99.109071) (end 128.299932 99.109) (width 0.2) (layer "B.Cu") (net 13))
 (segment (start 135 103.400057) (end 131.709943 100.11) (width 0.2) (layer "F.Cu") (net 11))
 (segment (start 131.709943 100.11) (end 126.25 100.11) (width 0.2) (layer "F.Cu") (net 11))
 (segment (start 135 108.05) (end 135 103.400057) (width 0.2) (layer "F.Cu") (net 11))
 (segment (start 129.100006 100.859994) (end 129.100006 100.71) (width 0.2) (layer "F.Cu") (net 14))
 (segment (start 131.65755 97.51) (end 132.567131 98.419581) (width 0.2) (layer "F.Cu") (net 14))
 (segment (start 132.567131 98.419581) (end 132.567131 98.984458) (width 0.2) (layer "F.Cu") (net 14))
 (segment (start 130.047 97.51) (end 131.65755 97.51) (width 0.2) (layer "F.Cu") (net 14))
 (segment (start 136.5 102.917327) (end 136.5 108.05) (width 0.2) (layer "F.Cu") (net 14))
 (segment (start 126.25 101.61) (end 126.982957 101.61) (width 0.2) (layer "F.Cu") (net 14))
 (segment (start 132.567131 98.984458) (end 136.5 102.917327) (width 0.2) (layer "F.Cu") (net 14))
 (segment (start 126.982957 101.61) (end 127.122957 101.75) (width 0.2) (layer "F.Cu") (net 14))
 (segment (start 127.122957 101.75) (end 128.21 101.75) (width 0.2) (layer "F.Cu") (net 14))
 (segment (start 128.21 101.75) (end 129.100006 100.859994) (width 0.2) (layer "F.Cu") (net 14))
 (segment (start 129.25 98.307) (end 130.047 97.51) (width 0.2) (layer "F.Cu") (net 14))
 (via (at 129.25 98.307) (size 0.6) (drill 0.3) (layers "F.Cu" "B.Cu") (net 14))
 (via (at 129.100006 100.71) (size 0.6) (drill 0.3) (layers "F.Cu" "B.Cu") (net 14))
 (segment (start 129.25 98.307) (end 129.25 100.560006) (width 0.2) (layer "B.Cu") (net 14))
 (segment (start 129.25 100.560006) (end 129.100006 100.71) (width 0.2) (layer "B.Cu") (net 14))
 (segment (start 128.4161 96.099) (end 127.5751 95.258) (width 0.2) (layer "F.Cu") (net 16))
 (segment (start 125.5309 102.61) (end 126.25 102.61) (width 0.2) (layer "F.Cu") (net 16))
 (segment (start 124.748998 96.128222) (end 124.748998 101.828098) (width 0.2) (layer "F.Cu") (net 16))
 (segment (start 132.016043 96.099) (end 137.5 101.582957) (width 0.2) (layer "F.Cu") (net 16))
 (segment (start 125.61922 95.258) (end 124.748998 96.128222) (width 0.2) (layer "F.Cu") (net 16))
 (segment (start 124.748998 101.828098) (end 125.5309 102.61) (width 0.2) (layer "F.Cu") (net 16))
 (segment (start 132.016043 96.099) (end 128.4161 96.099) (width 0.2) (layer "F.Cu") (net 16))
 (segment (start 127.5751 95.258) (end 125.61922 95.258) (width 0.2) (layer "F.Cu") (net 16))
 (segment (start 137.5 108.05) (end 137.5 101.582957) (width 0.2) (layer "F.Cu") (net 16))
 (segment (start 127.409 95.659) (end 125.78532 95.659) (width 0.2) (layer "F.Cu") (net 15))
 (segment (start 137 101.650057) (end 131.849943 96.5) (width 0.2) (layer "F.Cu") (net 15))
 (segment (start 137 108.05) (end 137 101.650057) (width 0.2) (layer "F.Cu") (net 15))
 (segment (start 125.349998 101.861998) (end 125.598 102.11) (width 0.2) (layer "F.Cu") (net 15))
 (segment (start 128.25 96.5) (end 127.409 95.659) (width 0.2) (layer "F.Cu") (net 15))
 (segment (start 131.849943 96.5) (end 128.25 96.5) (width 0.2) (layer "F.Cu") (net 15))
 (segment (start 125.349998 96.094322) (end 125.349998 101.861998) (width 0.2) (layer "F.Cu") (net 15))
 (segment (start 125.598 102.11) (end 126.25 102.11) (width 0.2) (layer "F.Cu") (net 15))
 (segment (start 125.78532 95.659) (end 125.349998 96.094322) (width 0.2) (layer "F.Cu") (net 15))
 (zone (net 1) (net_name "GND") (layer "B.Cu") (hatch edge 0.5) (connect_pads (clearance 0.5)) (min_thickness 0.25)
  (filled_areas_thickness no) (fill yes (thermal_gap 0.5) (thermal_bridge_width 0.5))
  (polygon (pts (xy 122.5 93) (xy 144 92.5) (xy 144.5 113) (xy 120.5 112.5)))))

